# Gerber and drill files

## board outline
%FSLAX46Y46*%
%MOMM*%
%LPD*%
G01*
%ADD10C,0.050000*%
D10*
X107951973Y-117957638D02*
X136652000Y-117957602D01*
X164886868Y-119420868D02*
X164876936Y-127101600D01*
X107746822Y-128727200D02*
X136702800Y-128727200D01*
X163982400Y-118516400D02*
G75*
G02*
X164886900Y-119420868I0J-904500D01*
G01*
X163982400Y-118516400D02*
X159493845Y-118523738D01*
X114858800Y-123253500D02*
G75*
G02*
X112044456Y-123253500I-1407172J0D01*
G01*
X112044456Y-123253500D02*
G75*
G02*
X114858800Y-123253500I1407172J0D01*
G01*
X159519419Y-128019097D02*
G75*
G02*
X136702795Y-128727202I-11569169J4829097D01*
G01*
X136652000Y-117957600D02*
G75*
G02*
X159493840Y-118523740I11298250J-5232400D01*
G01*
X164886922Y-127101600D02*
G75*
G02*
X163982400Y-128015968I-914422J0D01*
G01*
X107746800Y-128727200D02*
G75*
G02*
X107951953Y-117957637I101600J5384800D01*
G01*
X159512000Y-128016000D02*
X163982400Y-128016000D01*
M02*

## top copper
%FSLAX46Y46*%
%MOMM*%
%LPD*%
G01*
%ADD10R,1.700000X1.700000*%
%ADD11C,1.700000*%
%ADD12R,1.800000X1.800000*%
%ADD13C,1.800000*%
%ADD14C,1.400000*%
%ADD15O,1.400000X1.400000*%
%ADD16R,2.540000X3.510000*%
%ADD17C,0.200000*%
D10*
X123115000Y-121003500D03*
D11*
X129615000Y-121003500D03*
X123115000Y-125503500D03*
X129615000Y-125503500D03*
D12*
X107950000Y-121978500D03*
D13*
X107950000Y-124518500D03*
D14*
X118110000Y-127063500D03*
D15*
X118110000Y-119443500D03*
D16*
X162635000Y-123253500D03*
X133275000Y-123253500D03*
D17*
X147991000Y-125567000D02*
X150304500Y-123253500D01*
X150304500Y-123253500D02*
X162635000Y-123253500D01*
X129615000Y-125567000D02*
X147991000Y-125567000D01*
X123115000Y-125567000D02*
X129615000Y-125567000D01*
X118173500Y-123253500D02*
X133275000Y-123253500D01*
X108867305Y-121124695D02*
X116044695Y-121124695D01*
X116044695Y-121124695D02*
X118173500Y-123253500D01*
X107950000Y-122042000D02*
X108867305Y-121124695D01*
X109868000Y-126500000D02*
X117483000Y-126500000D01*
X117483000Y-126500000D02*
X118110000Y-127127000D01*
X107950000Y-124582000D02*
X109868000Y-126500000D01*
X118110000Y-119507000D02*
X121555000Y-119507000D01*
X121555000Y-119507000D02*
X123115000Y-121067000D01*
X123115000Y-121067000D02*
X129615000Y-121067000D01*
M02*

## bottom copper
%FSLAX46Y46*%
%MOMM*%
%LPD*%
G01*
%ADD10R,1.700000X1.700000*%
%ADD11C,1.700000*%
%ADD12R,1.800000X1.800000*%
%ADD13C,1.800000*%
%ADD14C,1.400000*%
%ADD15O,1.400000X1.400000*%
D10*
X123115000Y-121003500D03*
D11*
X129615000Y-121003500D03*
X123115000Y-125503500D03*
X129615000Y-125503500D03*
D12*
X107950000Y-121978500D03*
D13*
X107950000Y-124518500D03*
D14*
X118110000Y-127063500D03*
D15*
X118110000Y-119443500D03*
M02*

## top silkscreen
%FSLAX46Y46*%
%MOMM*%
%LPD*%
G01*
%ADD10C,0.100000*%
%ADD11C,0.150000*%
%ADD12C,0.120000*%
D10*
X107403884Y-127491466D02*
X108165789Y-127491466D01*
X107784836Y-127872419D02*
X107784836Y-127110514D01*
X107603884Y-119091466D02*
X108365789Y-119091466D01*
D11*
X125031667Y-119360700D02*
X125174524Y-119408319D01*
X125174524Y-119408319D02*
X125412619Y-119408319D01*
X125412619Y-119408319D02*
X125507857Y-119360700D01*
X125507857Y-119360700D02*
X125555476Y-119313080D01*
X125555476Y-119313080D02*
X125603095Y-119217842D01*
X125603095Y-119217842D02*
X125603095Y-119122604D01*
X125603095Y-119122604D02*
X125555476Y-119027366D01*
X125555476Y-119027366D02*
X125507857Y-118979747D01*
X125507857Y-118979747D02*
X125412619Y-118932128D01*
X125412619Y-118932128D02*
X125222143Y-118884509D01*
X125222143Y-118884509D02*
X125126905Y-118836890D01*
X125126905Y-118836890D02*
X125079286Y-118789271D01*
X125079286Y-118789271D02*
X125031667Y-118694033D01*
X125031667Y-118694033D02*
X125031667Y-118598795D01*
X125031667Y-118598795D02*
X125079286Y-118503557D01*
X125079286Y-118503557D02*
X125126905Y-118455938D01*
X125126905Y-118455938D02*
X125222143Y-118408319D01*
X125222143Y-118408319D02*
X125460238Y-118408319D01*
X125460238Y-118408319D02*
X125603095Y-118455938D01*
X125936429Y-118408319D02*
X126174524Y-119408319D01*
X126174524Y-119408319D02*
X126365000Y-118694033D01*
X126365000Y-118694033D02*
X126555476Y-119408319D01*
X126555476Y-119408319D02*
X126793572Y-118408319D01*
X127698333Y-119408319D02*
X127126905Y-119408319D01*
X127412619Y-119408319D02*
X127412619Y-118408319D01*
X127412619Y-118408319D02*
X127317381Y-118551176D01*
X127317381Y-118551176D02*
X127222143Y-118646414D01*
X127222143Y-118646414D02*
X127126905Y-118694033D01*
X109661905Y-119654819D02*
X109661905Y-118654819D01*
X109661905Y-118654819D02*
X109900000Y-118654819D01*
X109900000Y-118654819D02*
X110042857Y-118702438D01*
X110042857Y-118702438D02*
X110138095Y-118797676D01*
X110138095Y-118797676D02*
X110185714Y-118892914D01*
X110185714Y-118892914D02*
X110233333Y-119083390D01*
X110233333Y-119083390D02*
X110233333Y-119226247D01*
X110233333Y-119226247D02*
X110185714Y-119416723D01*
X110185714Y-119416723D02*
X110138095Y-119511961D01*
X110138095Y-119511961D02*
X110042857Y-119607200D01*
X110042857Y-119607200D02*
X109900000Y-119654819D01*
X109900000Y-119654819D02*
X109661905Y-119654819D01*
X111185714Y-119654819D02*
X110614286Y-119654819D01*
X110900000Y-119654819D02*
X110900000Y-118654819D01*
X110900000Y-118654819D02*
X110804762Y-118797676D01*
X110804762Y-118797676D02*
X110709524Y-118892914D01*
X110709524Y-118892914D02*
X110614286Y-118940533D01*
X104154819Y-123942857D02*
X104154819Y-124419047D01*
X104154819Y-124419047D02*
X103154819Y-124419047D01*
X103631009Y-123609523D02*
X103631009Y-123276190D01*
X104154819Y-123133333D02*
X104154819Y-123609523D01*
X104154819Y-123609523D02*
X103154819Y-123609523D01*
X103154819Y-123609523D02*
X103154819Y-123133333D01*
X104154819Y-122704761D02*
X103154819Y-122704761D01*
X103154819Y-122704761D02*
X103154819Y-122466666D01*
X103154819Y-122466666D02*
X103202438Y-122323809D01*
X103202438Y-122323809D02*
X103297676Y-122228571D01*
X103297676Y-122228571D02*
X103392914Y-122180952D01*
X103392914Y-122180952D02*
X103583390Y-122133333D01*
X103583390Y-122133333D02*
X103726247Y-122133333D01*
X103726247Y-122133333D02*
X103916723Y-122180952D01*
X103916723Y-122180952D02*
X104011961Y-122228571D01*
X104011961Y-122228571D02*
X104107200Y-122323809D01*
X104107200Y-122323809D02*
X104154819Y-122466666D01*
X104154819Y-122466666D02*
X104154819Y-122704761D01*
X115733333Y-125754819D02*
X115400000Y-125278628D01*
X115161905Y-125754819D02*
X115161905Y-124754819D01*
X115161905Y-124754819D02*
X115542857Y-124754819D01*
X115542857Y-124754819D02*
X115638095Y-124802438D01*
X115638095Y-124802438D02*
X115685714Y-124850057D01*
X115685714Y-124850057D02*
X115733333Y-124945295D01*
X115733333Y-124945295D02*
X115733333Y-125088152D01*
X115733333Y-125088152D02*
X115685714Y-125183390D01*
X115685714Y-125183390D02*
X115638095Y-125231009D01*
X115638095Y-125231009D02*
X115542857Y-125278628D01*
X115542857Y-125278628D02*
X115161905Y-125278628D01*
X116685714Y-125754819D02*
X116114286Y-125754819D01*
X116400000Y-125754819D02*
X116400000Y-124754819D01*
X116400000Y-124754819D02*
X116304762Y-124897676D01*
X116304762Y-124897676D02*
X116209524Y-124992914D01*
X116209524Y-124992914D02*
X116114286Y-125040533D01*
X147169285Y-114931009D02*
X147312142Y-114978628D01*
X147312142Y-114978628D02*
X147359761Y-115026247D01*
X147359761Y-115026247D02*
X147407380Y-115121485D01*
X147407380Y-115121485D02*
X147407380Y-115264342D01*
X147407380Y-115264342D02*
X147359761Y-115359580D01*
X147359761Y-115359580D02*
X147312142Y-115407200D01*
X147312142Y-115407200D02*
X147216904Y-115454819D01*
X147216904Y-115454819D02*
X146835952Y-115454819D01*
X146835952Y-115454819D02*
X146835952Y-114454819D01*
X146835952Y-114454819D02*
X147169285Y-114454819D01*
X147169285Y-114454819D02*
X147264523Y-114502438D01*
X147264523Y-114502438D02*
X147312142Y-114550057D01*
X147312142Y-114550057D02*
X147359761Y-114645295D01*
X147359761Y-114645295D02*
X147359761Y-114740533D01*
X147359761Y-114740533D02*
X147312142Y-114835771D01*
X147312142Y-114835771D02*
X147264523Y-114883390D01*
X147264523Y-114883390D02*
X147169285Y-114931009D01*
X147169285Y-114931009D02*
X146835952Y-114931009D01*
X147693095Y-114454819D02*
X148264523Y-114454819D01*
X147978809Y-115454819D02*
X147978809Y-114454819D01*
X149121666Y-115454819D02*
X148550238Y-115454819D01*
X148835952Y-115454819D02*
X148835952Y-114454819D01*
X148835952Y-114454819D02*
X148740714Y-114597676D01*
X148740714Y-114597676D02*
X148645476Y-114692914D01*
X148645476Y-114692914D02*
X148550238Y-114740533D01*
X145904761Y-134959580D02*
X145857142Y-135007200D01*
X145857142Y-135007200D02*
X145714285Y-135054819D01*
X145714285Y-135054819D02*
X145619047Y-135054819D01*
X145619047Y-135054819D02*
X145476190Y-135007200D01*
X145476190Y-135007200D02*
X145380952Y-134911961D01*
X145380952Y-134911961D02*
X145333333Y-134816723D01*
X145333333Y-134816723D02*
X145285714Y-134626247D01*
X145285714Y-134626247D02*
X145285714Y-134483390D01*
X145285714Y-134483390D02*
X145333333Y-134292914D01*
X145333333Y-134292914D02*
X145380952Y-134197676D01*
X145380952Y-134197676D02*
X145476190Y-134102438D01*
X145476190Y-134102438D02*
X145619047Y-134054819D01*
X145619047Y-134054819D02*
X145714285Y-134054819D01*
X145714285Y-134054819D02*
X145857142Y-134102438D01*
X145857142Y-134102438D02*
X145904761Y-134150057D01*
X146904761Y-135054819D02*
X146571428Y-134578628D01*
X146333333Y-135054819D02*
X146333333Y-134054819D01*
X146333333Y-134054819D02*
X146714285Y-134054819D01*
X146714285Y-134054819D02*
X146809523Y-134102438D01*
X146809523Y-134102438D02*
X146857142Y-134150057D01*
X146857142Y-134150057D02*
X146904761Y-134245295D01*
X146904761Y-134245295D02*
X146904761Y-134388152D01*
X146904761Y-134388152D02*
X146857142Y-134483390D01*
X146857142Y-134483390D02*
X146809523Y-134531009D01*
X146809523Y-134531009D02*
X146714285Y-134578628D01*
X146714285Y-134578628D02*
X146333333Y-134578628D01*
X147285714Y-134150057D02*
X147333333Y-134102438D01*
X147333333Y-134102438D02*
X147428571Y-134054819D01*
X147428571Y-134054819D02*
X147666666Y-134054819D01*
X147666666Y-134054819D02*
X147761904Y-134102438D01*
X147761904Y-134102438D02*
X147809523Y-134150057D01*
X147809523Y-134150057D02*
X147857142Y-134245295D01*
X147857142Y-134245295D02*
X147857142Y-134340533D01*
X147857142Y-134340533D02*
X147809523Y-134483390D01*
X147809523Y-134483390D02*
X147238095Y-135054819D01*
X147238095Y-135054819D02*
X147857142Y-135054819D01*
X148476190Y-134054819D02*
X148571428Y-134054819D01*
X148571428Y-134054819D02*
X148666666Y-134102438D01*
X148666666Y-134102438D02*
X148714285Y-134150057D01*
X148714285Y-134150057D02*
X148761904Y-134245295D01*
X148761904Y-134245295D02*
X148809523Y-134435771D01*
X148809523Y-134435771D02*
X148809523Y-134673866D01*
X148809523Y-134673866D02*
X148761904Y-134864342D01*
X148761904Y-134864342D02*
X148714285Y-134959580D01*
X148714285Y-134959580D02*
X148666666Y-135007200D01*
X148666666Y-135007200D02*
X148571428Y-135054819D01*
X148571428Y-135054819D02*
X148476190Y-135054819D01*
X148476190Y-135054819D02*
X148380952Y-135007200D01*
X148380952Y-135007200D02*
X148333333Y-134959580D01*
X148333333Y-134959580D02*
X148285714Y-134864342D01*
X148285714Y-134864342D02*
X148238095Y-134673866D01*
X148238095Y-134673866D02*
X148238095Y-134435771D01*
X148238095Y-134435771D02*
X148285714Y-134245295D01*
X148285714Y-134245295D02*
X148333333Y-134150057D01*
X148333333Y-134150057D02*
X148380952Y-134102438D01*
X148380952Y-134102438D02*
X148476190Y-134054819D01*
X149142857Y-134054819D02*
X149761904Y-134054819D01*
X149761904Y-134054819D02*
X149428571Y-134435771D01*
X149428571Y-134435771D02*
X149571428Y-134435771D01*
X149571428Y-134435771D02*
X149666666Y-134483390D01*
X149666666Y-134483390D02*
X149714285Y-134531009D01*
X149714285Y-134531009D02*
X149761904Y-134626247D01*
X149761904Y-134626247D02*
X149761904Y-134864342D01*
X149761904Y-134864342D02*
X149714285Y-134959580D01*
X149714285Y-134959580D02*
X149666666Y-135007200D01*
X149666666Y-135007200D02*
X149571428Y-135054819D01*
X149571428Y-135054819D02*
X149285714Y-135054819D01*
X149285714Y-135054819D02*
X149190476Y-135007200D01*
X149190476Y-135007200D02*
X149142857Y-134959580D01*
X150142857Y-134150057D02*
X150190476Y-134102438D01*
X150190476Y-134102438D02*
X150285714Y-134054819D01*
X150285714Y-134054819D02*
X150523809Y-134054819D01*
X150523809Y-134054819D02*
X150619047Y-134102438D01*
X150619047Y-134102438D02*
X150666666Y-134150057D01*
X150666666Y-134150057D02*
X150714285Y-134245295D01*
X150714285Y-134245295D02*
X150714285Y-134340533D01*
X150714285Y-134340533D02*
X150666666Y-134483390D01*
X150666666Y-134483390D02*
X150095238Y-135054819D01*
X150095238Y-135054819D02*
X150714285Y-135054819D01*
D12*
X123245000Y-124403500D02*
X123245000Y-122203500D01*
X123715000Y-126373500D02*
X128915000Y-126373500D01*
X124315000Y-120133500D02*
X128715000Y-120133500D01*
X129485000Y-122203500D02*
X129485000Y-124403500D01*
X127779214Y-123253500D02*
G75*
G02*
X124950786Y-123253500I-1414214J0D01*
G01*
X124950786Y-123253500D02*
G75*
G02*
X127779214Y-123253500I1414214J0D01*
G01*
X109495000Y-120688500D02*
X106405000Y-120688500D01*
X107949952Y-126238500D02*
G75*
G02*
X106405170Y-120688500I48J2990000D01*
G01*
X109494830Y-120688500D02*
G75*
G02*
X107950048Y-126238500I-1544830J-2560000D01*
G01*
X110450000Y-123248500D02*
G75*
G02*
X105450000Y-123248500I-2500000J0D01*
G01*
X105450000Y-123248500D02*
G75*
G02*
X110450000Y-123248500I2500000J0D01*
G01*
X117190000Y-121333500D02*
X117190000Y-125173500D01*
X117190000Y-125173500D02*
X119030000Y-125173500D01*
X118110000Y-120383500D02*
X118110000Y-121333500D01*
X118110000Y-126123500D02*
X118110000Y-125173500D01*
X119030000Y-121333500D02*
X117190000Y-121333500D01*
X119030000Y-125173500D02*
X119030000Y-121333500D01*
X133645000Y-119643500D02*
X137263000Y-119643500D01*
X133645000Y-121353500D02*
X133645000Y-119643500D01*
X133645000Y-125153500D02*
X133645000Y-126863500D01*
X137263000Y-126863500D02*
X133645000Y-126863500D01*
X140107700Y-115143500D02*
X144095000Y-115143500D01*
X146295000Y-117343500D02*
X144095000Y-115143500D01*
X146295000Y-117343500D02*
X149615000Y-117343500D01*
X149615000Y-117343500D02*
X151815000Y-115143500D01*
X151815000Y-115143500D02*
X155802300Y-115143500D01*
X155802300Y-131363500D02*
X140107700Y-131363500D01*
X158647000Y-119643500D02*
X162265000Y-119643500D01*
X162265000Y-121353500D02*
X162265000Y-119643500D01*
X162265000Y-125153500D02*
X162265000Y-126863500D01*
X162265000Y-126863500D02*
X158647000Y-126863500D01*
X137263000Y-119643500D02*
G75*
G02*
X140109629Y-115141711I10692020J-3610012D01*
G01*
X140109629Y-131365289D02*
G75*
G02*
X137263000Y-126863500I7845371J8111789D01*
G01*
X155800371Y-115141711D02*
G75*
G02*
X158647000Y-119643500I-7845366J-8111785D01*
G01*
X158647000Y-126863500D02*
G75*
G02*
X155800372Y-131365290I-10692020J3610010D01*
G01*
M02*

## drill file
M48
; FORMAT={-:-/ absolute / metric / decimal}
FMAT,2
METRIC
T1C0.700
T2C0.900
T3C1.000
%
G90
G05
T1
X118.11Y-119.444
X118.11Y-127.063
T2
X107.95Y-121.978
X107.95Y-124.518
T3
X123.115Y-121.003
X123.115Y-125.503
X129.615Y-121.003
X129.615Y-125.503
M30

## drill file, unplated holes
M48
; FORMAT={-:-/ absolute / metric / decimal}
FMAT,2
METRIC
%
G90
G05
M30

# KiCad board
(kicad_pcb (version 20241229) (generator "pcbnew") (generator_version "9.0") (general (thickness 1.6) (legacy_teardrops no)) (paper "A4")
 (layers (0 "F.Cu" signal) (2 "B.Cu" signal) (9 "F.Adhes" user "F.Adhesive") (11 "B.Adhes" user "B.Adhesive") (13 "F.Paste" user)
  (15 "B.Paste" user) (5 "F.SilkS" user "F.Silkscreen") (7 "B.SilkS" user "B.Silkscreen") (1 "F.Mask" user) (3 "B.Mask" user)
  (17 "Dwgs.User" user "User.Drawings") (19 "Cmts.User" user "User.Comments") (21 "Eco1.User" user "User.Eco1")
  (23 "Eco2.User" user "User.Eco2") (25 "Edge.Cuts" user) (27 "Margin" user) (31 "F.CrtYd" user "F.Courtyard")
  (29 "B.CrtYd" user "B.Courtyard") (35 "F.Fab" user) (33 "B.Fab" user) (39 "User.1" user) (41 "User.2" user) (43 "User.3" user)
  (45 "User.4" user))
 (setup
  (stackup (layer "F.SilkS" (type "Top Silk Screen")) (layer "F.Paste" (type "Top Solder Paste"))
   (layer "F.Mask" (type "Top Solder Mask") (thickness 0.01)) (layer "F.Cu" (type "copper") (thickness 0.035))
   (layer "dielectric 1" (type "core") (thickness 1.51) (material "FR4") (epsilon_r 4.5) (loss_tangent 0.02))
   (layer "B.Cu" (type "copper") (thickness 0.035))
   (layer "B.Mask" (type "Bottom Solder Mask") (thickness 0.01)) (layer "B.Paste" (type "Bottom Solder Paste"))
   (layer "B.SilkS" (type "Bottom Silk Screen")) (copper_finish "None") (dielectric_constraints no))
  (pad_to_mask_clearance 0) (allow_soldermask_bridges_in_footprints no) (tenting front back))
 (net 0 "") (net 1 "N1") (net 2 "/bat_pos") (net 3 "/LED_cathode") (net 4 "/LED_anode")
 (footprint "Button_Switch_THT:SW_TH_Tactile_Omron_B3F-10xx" (layer "F.Cu") (at 123.115 121.0035)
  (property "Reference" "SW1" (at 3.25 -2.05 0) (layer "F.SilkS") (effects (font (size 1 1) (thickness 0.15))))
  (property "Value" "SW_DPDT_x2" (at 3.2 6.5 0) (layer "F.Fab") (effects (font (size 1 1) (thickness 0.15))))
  (fp_line (start 0.13 3.4) (end 0.13 1.2) (stroke (width 0.12) (type solid)) (layer "F.SilkS"))
  (fp_line (start 0.6 5.37) (end 5.8 5.37) (stroke (width 0.12) (type solid)) (layer "F.SilkS"))
  (fp_line (start 1.2 -0.87) (end 5.6 -0.87) (stroke (width 0.12) (type solid)) (layer "F.SilkS"))
  (fp_line (start 6.37 1.2) (end 6.37 3.4) (stroke (width 0.12) (type solid)) (layer "F.SilkS"))
  (fp_circle (center 3.25 2.25) (end 4.25 3.25) (stroke (width 0.12) (type solid)) (fill no) (layer "F.SilkS"))
  (pad "1" thru_hole rect (at 0 0) (size 1.7 1.7) (drill 1) (layers "*.Cu" "*.Mask") (remove_unused_layers no) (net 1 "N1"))
  (pad "1" thru_hole circle (at 6.5 0) (size 1.7 1.7) (drill 1) (layers "*.Cu" "*.Mask") (remove_unused_layers no) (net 1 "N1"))
  (pad "2" thru_hole circle (at 0 4.5) (size 1.7 1.7) (drill 1) (layers "*.Cu" "*.Mask") (remove_unused_layers no) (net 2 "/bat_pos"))
  (pad "2" thru_hole circle (at 6.5 4.5) (size 1.7 1.7) (drill 1) (layers "*.Cu" "*.Mask") (remove_unused_layers no) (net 2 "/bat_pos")))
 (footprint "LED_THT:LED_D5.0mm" (layer "F.Cu") (at 107.95 121.9785 -90)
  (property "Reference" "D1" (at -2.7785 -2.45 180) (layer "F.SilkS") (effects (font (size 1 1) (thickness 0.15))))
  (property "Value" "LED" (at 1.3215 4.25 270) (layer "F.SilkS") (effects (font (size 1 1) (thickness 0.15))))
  (fp_line (start -1.29 -1.545) (end -1.29 1.545) (stroke (width 0.12) (type solid)) (layer "F.SilkS"))
  (fp_arc (start 4.26 0.000048) (mid 2.071756 2.880501) (end -1.29 1.54483) (stroke (width 0.12) (type solid)) (layer "F.SilkS"))
  (fp_arc (start -1.29 -1.54483) (mid 2.071756 -2.880501) (end 4.26 -0.000048) (stroke (width 0.12) (type solid)) (layer "F.SilkS"))
  (fp_circle (center 1.27 0) (end 3.77 0) (stroke (width 0.12) (type solid)) (fill no) (layer "F.SilkS"))
  (pad "1" thru_hole rect (at 0 0 270) (size 1.8 1.8) (drill 0.9) (layers "*.Cu" "*.Mask") (remove_unused_layers no) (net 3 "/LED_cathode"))
  (pad "2" thru_hole circle (at 2.54 0 270) (size 1.8 1.8) (drill 0.9) (layers "*.Cu" "*.Mask") (remove_unused_layers no)
   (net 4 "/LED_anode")))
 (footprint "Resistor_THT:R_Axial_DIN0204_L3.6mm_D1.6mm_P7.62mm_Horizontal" (layer "F.Cu") (at 118.11 127.0635 90)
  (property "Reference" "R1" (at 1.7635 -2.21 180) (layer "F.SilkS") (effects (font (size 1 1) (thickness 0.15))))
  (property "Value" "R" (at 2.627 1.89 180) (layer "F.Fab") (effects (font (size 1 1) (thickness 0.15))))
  (fp_line (start 5.73 -0.92) (end 1.89 -0.92) (stroke (width 0.12) (type solid)) (layer "F.SilkS"))
  (fp_line (start 1.89 -0.92) (end 1.89 0.92) (stroke (width 0.12) (type solid)) (layer "F.SilkS"))
  (fp_line (start 6.68 0) (end 5.73 0) (stroke (width 0.12) (type solid)) (layer "F.SilkS"))
  (fp_line (start 0.94 0) (end 1.89 0) (stroke (width 0.12) (type solid)) (layer "F.SilkS"))
  (fp_line (start 5.73 0.92) (end 5.73 -0.92) (stroke (width 0.12) (type solid)) (layer "F.SilkS"))
  (fp_line (start 1.89 0.92) (end 5.73 0.92) (stroke (width 0.12) (type solid)) (layer "F.SilkS"))
  (pad "1" thru_hole circle (at 0 0 90) (size 1.4 1.4) (drill 0.7) (layers "*.Cu" "*.Mask") (remove_unused_layers no) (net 4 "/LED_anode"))
  (pad "2" thru_hole oval (at 7.62 0 90) (size 1.4 1.4) (drill 0.7) (layers "*.Cu" "*.Mask") (remove_unused_layers no) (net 1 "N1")))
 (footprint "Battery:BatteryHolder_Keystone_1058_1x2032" (layer "F.Cu") (at 147.955 123.2535 180)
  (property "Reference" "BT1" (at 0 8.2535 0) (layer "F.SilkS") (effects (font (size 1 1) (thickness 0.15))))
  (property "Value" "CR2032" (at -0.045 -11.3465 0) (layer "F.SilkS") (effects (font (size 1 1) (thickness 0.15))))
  (fp_line (start 14.31 3.61) (end 10.692 3.61) (stroke (width 0.12) (type solid)) (layer "F.SilkS"))
  (fp_line (start 14.31 1.9) (end 14.31 3.61) (stroke (width 0.12) (type solid)) (layer "F.SilkS"))
  (fp_line (start 14.31 -1.9) (end 14.31 -3.61) (stroke (width 0.12) (type solid)) (layer "F.SilkS"))
  (fp_line (start 10.692 -3.61) (end 14.31 -3.61) (stroke (width 0.12) (type solid)) (layer "F.SilkS"))
  (fp_line (start 7.8473 8.11) (end 3.86 8.11) (stroke (width 0.12) (type solid)) (layer "F.SilkS"))
  (fp_line (start 1.66 5.91) (end 3.86 8.11) (stroke (width 0.12) (type solid)) (layer "F.SilkS"))
  (fp_line (start 1.66 5.91) (end -1.66 5.91) (stroke (width 0.12) (type solid)) (layer "F.SilkS"))
  (fp_line (start -1.66 5.91) (end -3.86 8.11) (stroke (width 0.12) (type solid)) (layer "F.SilkS"))
  (fp_line (start -3.86 8.11) (end -7.8473 8.11) (stroke (width 0.12) (type solid)) (layer "F.SilkS"))
  (fp_line (start -7.8473 -8.11) (end 7.8473 -8.11) (stroke (width 0.12) (type solid)) (layer "F.SilkS"))
  (fp_line (start -10.692 3.61) (end -14.31 3.61) (stroke (width 0.12) (type solid)) (layer "F.SilkS"))
  (fp_line (start -14.31 1.9) (end -14.31 3.61) (stroke (width 0.12) (type solid)) (layer "F.SilkS"))
  (fp_line (start -14.31 -1.9) (end -14.31 -3.61) (stroke (width 0.12) (type solid)) (layer "F.SilkS"))
  (fp_line (start -14.31 -3.61) (end -10.692 -3.61) (stroke (width 0.12) (type solid)) (layer "F.SilkS"))
  (fp_arc (start 10.692 3.61) (mid 9.538084 6.031244) (end 7.845371 8.111789) (stroke (width 0.12) (type solid)) (layer "F.SilkS"))
  (fp_arc (start 7.845371 -8.111789) (mid 9.538085 -6.031244) (end 10.692 -3.61) (stroke (width 0.12) (type solid)) (layer "F.SilkS"))
  (fp_arc (start -7.845371 8.111789) (mid -9.538085 6.031244) (end -10.692 3.61) (stroke (width 0.12) (type solid)) (layer "F.SilkS"))
  (fp_arc (start -10.692 -3.61) (mid -9.538084 -6.031244) (end -7.845371 -8.111789) (stroke (width 0.12) (type solid)) (layer "F.SilkS"))
  (pad "1" smd rect (at -14.68 0 180) (size 2.54 3.51) (layers "F.Cu" "F.Mask" "F.Paste") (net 2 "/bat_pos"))
  (pad "2" smd rect (at 14.68 0 180) (size 2.54 3.51) (layers "F.Cu" "F.Mask" "F.Paste") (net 3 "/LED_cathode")))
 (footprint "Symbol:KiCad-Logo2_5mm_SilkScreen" (layer "B.Cu") (at 148.59 119.38 180)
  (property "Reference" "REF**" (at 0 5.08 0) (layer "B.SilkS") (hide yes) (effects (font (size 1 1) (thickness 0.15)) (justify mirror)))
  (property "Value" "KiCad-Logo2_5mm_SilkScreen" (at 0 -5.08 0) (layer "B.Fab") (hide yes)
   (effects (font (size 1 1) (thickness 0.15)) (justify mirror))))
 (gr_line (start 107.951973 117.957638) (end 136.652 117.957602) (stroke (width 0.05) (type default)) (layer "Edge.Cuts"))
 (gr_line (start 164.886868 119.420868) (end 164.876936 127.1016) (stroke (width 0.05) (type default)) (layer "Edge.Cuts"))
 (gr_line (start 107.746822 128.7272) (end 136.7028 128.7272) (stroke (width 0.05) (type default)) (layer "Edge.Cuts"))
 (gr_arc (start 163.9824 118.5164) (mid 164.621955 118.781313) (end 164.886868 119.420868) (stroke (width 0.05) (type default))
  (layer "Edge.Cuts"))
 (gr_line (start 163.9824 118.5164) (end 159.493845 118.523738) (stroke (width 0.05) (type default)) (layer "Edge.Cuts"))
 (gr_circle (center 113.451628 123.2535) (end 114.213628 124.4365) (stroke (width 0.05) (type default)) (fill no) (layer "Edge.Cuts"))
 (gr_arc (start 159.519419 128.019097) (mid 148.339133 135.720545) (end 136.7028 128.7272) (stroke (width 0.05) (type default))
  (layer "Edge.Cuts"))
 (gr_arc (start 136.652 117.9576) (mid 148.258759 110.742777) (end 159.493845 118.523738) (stroke (width 0.05) (type default))
  (layer "Edge.Cuts"))
 (gr_arc (start 164.886922 127.1016) (mid 164.622586 127.744695) (end 163.9824 128.016) (stroke (width 0.05) (type default))
  (layer "Edge.Cuts"))
 (gr_arc (start 107.7468 128.7272) (mid 102.463619 123.239823) (end 107.951953 117.957638) (stroke (width 0.05) (type default))
  (layer "Edge.Cuts"))
 (gr_line (start 159.512 128.016) (end 163.9824 128.016) (stroke (width 0.05) (type default)) (layer "Edge.Cuts"))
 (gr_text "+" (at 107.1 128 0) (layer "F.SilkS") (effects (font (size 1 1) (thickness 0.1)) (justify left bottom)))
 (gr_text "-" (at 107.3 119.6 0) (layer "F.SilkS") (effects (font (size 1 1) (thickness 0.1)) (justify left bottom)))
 (segment (start 147.991 125.567) (end 150.3045 123.2535) (width 0.2) (layer "F.Cu") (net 2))
 (segment (start 150.3045 123.2535) (end 162.635 123.2535) (width 0.2) (layer "F.Cu") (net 2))
 (segment (start 129.615 125.567) (end 147.991 125.567) (width 0.2) (layer "F.Cu") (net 2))
 (segment (start 123.115 125.567) (end 129.615 125.567) (width 0.2) (layer "F.Cu") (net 2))
 (segment (start 118.1735 123.2535) (end 133.275 123.2535) (width 0.2) (layer "F.Cu") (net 3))
 (segment (start 108.867305 121.124695) (end 116.044695 121.124695) (width 0.2) (layer "F.Cu") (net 3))
 (segment (start 116.044695 121.124695) (end 118.1735 123.2535) (width 0.2) (layer "F.Cu") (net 3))
 (segment (start 107.95 122.042) (end 108.867305 121.124695) (width 0.2) (layer "F.Cu") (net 3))
 (segment (start 109.868 126.5) (end 117.483 126.5) (width 0.2) (layer "F.Cu") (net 4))
 (segment (start 117.483 126.5) (end 118.11 127.127) (width 0.2) (layer "F.Cu") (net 4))
 (segment (start 107.95 124.582) (end 109.868 126.5) (width 0.2) (layer "F.Cu") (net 4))
 (segment (start 118.11 119.507) (end 121.555 119.507) (width 0.2) (layer "F.Cu") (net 1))
 (segment (start 121.555 119.507) (end 123.115 121.067) (width 0.2) (layer "F.Cu") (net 1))
 (segment (start 123.115 121.067) (end 129.615 121.067) (width 0.2) (layer "F.Cu") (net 1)))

